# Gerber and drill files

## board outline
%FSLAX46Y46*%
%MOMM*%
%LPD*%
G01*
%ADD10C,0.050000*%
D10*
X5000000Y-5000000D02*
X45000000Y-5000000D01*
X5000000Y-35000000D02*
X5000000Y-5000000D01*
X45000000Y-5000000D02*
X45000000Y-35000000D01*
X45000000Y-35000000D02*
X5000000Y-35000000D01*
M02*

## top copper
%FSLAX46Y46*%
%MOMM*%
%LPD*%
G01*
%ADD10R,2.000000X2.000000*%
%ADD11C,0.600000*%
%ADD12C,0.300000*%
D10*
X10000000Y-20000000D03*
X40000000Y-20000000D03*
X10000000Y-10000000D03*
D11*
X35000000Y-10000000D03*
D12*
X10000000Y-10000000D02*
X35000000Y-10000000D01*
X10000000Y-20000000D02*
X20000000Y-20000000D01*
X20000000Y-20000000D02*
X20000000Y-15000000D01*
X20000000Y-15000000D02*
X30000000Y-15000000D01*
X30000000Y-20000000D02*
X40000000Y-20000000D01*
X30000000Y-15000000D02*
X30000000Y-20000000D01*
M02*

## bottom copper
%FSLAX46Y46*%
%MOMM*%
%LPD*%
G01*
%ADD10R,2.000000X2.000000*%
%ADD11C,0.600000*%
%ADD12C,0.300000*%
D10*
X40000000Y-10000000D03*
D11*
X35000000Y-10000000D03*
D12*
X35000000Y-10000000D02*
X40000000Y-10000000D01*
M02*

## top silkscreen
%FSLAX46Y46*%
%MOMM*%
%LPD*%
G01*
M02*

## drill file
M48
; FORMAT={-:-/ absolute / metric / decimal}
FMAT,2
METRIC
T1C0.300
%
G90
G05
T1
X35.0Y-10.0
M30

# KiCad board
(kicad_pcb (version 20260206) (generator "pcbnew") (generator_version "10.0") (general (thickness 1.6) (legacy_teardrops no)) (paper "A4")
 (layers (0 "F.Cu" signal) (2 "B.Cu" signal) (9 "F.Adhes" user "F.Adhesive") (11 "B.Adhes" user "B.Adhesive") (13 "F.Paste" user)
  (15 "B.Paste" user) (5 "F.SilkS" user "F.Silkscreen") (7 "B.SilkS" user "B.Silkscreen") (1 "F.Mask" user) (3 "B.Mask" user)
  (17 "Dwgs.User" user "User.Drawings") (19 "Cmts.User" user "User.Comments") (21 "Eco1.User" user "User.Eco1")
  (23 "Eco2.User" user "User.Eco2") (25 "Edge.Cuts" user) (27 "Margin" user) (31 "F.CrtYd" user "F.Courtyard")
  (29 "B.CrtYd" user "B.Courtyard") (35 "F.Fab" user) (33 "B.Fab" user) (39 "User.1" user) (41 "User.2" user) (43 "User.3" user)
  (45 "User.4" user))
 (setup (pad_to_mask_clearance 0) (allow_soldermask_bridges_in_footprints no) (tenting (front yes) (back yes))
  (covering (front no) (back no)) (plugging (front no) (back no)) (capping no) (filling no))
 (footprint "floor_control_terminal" (layer "F.Cu") (at 10 20)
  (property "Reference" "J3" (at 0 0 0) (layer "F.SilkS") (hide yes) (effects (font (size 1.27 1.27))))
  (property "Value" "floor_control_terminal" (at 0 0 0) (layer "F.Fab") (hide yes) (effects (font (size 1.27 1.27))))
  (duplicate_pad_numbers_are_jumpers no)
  (pad "1" smd rect (at 0 0) (size 2 2) (layers "F.Cu" "F.Mask" "F.Paste") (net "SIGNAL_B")))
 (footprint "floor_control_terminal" (layer "F.Cu") (at 40 20)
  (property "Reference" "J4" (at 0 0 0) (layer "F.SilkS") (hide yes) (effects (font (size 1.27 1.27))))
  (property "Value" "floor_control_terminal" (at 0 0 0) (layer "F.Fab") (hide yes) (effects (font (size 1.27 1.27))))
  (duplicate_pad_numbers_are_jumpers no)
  (pad "1" smd rect (at 0 0) (size 2 2) (layers "F.Cu" "F.Mask" "F.Paste") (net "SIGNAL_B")))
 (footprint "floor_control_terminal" (layer "F.Cu") (at 10 10)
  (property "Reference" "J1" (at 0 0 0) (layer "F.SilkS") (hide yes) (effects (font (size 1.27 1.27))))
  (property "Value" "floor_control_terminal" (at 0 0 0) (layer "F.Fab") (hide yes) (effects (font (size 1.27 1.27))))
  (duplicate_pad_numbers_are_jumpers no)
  (pad "1" smd rect (at 0 0) (size 2 2) (layers "F.Cu" "F.Mask" "F.Paste") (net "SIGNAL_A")))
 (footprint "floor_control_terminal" (layer "B.Cu") (at 40 10)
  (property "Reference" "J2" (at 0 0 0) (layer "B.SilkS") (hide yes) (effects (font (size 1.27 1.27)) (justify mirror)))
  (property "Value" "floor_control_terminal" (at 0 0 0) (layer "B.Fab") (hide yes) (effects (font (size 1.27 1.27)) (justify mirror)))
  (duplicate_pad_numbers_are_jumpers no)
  (pad "1" smd rect (at 0 0) (size 2 2) (layers "B.Cu" "B.Mask" "B.Paste") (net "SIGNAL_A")))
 (gr_line (start 5 5) (end 45 5) (stroke (width 0.05) (type default)) (layer "Edge.Cuts"))
 (gr_line (start 5 35) (end 5 5) (stroke (width 0.05) (type default)) (layer "Edge.Cuts"))
 (gr_line (start 45 5) (end 45 35) (stroke (width 0.05) (type default)) (layer "Edge.Cuts"))
 (gr_line (start 45 35) (end 5 35) (stroke (width 0.05) (type default)) (layer "Edge.Cuts"))
 (segment (start 10 10) (end 35 10) (width 0.3) (layer "F.Cu") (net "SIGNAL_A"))
 (via (at 35 10) (size 0.6) (drill 0.3) (layers "F.Cu" "B.Cu") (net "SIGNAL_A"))
 (segment (start 35 10) (end 40 10) (width 0.3) (layer "B.Cu") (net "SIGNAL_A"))
 (segment (start 10 20) (end 20 20) (width 0.3) (layer "F.Cu") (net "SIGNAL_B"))
 (segment (start 20 20) (end 20 15) (width 0.3) (layer "F.Cu") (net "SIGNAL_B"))
 (segment (start 20 15) (end 30 15) (width 0.3) (layer "F.Cu") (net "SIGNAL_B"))
 (segment (start 30 20) (end 40 20) (width 0.3) (layer "F.Cu") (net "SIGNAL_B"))
 (segment (start 30 15) (end 30 20) (width 0.3) (layer "F.Cu") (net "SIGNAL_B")))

